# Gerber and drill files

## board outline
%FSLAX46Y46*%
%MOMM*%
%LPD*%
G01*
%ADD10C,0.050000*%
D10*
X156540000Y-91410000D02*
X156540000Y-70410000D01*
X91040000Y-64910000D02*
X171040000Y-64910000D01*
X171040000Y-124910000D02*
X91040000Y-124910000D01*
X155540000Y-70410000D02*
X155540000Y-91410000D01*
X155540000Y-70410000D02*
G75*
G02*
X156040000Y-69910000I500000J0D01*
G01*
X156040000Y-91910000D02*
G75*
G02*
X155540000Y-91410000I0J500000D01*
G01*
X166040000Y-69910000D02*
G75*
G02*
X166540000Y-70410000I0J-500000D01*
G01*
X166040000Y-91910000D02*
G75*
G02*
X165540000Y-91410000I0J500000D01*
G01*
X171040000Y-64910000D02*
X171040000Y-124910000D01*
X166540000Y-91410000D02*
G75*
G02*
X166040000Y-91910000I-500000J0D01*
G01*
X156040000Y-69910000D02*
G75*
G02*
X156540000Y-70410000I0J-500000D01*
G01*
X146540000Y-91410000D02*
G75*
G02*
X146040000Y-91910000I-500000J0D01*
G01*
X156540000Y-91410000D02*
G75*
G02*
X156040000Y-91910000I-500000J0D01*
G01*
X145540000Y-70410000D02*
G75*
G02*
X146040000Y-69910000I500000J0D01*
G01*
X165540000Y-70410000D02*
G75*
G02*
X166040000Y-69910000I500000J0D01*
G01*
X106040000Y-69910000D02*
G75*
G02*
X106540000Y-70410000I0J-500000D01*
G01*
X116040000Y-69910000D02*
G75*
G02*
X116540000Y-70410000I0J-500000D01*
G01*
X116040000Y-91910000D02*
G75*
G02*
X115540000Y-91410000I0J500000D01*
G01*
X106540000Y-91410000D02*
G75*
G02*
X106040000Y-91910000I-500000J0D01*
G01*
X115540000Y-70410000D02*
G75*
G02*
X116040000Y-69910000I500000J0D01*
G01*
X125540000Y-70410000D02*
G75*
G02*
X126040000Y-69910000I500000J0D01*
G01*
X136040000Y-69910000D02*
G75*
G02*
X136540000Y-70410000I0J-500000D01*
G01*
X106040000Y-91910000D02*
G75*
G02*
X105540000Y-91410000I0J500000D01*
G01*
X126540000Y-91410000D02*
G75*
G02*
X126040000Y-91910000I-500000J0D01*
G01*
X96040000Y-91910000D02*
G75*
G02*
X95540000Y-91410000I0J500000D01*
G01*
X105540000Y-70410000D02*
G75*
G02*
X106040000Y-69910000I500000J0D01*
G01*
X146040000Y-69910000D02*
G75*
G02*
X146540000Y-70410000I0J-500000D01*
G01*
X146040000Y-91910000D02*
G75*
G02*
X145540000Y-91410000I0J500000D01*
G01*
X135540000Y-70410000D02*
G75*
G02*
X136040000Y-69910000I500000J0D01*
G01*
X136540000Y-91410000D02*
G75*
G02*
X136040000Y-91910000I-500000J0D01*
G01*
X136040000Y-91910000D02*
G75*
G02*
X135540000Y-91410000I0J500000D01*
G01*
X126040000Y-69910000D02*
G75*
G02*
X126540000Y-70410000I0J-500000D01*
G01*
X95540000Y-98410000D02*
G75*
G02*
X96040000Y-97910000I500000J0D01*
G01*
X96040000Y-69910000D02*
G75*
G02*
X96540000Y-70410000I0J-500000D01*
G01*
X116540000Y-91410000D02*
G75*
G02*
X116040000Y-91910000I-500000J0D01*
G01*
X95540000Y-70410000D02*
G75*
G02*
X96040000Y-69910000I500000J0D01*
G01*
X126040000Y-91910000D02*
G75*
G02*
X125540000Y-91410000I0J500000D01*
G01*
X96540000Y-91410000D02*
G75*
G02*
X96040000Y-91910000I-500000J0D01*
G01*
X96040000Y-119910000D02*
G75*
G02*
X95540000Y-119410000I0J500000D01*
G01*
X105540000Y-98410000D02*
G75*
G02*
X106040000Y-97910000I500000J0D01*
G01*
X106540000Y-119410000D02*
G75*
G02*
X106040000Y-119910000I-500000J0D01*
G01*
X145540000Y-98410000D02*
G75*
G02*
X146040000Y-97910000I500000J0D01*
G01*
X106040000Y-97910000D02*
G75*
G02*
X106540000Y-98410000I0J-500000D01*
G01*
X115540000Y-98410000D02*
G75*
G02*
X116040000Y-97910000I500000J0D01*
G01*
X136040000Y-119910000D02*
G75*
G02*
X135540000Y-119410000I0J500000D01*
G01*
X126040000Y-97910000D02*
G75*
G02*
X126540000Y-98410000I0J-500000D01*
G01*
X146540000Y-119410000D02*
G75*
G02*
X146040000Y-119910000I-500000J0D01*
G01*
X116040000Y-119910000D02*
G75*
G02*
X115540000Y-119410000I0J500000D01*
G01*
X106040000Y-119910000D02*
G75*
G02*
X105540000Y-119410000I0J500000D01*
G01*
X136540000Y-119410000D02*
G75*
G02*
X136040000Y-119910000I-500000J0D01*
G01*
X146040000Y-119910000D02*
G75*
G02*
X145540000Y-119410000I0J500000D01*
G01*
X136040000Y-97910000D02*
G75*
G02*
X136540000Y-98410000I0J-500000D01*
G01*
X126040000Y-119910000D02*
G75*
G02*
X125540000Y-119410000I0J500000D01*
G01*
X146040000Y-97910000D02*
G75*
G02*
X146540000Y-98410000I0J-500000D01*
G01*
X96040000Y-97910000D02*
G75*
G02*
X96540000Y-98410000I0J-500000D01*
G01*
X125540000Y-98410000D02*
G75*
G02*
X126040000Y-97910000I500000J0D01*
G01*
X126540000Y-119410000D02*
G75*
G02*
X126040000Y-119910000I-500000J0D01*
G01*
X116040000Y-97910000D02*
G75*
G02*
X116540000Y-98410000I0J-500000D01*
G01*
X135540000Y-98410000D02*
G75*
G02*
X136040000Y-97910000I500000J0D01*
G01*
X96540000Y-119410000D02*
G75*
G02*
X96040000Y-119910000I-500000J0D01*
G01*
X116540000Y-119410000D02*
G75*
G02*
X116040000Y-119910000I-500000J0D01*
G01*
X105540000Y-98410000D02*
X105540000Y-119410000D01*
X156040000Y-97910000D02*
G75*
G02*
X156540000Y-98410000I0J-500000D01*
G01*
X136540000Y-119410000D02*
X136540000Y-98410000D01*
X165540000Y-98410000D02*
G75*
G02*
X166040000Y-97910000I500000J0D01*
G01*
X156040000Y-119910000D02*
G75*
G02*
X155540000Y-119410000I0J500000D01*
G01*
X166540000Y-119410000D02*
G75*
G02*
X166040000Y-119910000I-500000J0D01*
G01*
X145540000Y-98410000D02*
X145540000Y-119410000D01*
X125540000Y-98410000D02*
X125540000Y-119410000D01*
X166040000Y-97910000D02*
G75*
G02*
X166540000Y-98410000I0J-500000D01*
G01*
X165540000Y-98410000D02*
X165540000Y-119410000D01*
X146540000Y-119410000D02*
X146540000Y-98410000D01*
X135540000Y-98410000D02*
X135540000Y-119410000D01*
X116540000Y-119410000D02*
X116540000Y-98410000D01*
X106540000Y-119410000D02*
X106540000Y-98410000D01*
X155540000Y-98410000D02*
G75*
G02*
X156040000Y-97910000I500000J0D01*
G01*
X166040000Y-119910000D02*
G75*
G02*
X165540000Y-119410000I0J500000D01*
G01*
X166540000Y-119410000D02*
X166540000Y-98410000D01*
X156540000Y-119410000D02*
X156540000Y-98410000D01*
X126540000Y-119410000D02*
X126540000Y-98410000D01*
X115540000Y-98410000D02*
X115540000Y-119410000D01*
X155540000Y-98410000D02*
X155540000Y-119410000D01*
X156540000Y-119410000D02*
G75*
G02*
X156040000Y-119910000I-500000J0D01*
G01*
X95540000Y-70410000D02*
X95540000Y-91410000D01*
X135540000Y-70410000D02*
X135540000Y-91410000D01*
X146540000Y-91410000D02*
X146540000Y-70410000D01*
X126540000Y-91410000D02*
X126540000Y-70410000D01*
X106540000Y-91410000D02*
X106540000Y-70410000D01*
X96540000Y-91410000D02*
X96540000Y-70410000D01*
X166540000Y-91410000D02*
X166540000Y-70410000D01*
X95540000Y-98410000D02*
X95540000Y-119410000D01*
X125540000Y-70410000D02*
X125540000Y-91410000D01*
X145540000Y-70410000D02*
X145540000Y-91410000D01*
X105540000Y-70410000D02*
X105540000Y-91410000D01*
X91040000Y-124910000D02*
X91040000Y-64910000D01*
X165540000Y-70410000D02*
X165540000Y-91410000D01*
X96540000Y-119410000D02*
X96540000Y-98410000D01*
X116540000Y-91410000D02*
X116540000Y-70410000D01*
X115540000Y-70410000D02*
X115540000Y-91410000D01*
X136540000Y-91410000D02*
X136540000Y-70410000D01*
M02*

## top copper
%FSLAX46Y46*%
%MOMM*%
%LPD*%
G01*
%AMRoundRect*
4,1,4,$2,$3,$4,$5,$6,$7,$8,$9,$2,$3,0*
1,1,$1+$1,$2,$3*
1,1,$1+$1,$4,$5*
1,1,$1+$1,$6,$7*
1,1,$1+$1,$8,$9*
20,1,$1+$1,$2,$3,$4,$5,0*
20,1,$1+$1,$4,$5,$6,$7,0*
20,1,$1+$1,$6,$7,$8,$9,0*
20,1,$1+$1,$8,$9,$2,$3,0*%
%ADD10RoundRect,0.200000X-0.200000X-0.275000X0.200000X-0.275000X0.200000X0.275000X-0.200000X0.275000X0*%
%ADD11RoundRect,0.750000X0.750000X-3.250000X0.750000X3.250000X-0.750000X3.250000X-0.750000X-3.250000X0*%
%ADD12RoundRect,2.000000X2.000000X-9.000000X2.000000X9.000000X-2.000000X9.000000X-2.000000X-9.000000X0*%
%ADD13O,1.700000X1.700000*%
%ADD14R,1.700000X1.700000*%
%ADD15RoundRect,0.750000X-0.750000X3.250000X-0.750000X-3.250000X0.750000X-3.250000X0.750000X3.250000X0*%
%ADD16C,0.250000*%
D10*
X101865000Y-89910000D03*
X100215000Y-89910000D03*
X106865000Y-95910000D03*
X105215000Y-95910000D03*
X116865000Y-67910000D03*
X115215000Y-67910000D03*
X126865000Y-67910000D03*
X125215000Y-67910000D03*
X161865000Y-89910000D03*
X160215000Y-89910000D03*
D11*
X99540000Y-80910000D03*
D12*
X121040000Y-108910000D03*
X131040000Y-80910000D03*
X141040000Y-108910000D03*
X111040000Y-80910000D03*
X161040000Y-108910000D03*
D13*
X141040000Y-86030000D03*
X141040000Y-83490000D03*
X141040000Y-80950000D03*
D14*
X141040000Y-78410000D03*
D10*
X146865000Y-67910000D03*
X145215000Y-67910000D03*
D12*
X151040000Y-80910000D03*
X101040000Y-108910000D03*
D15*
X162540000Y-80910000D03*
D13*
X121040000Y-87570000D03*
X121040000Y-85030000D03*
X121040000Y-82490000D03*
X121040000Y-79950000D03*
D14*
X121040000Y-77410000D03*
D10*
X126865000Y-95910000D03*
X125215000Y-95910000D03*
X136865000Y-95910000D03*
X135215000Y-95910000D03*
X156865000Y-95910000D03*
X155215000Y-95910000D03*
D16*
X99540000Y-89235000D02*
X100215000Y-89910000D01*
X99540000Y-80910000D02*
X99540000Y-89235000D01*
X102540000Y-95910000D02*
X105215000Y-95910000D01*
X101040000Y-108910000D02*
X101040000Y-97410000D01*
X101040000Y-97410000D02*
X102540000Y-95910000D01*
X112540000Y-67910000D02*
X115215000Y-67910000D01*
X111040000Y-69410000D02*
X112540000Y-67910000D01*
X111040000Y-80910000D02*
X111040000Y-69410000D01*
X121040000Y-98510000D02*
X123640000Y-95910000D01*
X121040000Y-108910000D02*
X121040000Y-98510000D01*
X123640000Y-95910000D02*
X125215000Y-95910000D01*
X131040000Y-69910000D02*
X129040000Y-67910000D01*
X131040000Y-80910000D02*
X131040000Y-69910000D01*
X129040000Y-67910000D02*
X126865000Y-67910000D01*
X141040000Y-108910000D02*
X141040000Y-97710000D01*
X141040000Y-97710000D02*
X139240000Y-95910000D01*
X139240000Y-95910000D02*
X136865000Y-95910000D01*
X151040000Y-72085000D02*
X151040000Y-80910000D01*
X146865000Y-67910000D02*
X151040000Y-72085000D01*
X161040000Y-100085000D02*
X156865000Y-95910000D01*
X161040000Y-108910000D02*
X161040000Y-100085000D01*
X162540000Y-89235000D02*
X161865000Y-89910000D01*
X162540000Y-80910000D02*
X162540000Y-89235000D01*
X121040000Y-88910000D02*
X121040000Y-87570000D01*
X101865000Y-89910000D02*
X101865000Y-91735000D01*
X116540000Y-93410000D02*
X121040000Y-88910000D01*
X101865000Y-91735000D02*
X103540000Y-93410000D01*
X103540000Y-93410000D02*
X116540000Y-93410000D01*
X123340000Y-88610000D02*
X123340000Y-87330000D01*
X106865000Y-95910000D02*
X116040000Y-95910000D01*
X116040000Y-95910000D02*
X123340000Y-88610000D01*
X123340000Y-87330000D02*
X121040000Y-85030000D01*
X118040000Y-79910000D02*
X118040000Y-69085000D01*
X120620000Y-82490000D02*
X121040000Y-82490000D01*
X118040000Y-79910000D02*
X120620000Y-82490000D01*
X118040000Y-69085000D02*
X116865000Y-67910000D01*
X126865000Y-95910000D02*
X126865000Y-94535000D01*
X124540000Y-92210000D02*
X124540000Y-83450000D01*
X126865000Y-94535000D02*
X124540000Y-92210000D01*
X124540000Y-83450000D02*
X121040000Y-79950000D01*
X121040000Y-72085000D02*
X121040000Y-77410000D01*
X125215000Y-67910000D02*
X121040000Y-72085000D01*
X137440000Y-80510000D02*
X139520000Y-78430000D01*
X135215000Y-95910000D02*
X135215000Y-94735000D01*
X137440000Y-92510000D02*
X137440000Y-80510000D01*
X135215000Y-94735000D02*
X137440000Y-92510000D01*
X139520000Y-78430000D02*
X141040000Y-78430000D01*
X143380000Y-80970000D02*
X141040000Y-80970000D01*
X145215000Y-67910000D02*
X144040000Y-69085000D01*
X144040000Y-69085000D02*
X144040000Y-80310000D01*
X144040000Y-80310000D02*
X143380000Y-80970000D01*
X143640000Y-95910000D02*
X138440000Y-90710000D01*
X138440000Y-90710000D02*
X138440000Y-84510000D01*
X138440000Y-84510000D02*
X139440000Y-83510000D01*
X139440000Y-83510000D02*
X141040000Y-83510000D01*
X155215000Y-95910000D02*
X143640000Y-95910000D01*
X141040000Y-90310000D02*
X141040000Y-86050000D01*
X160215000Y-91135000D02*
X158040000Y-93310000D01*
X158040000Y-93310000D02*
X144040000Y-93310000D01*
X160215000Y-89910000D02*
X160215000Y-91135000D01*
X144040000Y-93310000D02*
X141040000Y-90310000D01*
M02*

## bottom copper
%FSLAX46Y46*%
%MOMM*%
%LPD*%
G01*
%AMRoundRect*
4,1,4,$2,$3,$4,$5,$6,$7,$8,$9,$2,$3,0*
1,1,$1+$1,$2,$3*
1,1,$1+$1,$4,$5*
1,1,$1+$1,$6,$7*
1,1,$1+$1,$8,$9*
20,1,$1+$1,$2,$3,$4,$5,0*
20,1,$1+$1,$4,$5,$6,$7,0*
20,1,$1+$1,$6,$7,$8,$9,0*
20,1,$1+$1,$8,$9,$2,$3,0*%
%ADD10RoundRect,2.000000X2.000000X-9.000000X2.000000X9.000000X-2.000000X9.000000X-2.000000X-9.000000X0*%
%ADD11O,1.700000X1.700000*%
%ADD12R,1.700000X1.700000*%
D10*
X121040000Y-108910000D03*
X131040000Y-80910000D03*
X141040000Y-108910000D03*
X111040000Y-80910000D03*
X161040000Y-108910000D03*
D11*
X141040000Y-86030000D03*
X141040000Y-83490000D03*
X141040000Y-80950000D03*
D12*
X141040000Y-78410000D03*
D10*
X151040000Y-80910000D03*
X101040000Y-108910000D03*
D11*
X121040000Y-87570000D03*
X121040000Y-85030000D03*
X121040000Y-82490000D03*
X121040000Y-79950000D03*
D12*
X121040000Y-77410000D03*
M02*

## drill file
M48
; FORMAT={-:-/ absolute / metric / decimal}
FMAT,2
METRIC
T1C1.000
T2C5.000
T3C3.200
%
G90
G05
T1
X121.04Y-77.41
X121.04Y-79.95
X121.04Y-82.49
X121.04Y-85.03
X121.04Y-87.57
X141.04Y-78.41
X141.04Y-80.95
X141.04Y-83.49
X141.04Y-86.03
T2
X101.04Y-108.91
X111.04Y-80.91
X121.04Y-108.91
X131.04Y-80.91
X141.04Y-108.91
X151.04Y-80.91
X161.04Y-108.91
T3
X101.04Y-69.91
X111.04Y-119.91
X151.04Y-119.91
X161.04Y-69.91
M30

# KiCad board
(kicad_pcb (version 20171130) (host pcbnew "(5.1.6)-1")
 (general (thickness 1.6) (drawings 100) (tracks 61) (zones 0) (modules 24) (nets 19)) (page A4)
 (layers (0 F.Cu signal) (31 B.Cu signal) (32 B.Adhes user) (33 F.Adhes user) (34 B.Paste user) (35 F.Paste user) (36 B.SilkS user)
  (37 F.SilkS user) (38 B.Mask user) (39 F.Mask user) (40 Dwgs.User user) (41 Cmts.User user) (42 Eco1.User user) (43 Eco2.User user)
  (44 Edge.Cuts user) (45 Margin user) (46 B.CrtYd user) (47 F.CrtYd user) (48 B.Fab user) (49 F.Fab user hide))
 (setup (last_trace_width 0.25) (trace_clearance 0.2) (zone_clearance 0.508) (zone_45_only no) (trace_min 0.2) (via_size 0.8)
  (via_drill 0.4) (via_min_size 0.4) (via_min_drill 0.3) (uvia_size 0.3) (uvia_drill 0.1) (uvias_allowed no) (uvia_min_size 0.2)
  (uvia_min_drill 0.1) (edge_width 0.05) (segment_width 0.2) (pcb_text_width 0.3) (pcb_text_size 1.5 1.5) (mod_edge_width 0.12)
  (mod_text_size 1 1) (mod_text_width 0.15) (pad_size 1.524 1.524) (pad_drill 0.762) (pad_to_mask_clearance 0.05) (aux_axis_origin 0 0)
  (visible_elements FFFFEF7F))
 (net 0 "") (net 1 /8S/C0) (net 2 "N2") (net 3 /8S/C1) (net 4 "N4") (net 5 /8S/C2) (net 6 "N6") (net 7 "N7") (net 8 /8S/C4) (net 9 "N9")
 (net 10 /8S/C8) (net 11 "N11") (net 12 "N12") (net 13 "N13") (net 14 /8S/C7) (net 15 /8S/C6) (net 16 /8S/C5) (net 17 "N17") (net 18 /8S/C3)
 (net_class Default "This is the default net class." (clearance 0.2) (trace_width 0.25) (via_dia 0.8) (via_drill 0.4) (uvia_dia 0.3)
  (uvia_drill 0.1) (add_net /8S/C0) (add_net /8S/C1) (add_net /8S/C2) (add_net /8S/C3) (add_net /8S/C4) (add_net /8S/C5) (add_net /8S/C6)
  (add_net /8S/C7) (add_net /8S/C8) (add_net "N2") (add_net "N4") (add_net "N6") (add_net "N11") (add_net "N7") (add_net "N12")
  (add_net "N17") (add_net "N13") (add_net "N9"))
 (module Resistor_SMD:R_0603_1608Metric (layer F.Cu) (at 101.04 89.91)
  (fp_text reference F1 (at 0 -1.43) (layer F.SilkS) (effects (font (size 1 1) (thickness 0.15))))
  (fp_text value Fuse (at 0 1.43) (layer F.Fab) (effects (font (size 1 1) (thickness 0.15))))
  (pad 2 smd roundrect (at 0.825 0) (size 0.8 0.95) (layers F.Cu F.Paste F.Mask) (roundrect_rratio 0.25) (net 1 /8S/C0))
  (pad 1 smd roundrect (at -0.825 0) (size 0.8 0.95) (layers F.Cu F.Paste F.Mask) (roundrect_rratio 0.25) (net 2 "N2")))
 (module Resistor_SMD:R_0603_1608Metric (layer F.Cu) (at 106.04 95.91)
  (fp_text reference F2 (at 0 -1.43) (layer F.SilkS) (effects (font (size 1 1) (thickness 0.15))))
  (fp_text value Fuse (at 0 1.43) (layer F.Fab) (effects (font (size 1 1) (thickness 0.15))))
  (pad 2 smd roundrect (at 0.825 0) (size 0.8 0.95) (layers F.Cu F.Paste F.Mask) (roundrect_rratio 0.25) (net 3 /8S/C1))
  (pad 1 smd roundrect (at -0.825 0) (size 0.8 0.95) (layers F.Cu F.Paste F.Mask) (roundrect_rratio 0.25) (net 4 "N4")))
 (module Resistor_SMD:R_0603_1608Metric (layer F.Cu) (at 116.04 67.91)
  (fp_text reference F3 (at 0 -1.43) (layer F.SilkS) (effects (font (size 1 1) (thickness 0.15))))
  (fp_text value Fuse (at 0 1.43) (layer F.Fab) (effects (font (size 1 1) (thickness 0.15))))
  (pad 2 smd roundrect (at 0.825 0) (size 0.8 0.95) (layers F.Cu F.Paste F.Mask) (roundrect_rratio 0.25) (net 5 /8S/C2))
  (pad 1 smd roundrect (at -0.825 0) (size 0.8 0.95) (layers F.Cu F.Paste F.Mask) (roundrect_rratio 0.25) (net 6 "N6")))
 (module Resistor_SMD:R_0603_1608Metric (layer F.Cu) (at 126.04 67.91)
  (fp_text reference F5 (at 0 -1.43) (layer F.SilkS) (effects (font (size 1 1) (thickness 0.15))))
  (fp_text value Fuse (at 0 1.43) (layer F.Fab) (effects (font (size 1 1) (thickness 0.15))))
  (pad 2 smd roundrect (at 0.825 0) (size 0.8 0.95) (layers F.Cu F.Paste F.Mask) (roundrect_rratio 0.25) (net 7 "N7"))
  (pad 1 smd roundrect (at -0.825 0) (size 0.8 0.95) (layers F.Cu F.Paste F.Mask) (roundrect_rratio 0.25) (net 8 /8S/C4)))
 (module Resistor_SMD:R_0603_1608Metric (layer F.Cu) (at 161.04 89.91)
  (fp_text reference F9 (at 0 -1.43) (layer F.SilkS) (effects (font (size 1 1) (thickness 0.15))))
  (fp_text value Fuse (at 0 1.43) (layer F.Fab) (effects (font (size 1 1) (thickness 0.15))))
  (pad 2 smd roundrect (at 0.825 0) (size 0.8 0.95) (layers F.Cu F.Paste F.Mask) (roundrect_rratio 0.25) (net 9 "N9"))
  (pad 1 smd roundrect (at -0.825 0) (size 0.8 0.95) (layers F.Cu F.Paste F.Mask) (roundrect_rratio 0.25) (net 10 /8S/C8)))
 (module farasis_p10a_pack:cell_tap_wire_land (layer F.Cu) (at 99.54 80.91 90)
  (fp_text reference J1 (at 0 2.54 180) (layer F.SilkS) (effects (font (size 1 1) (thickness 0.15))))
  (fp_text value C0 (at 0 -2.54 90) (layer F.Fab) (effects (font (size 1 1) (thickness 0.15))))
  (pad 1 smd roundrect (at 0 0 90) (size 8 3) (layers F.Cu F.Paste F.Mask) (roundrect_rratio 0.25) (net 2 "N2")))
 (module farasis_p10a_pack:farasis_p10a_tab (layer F.Cu) (at 121.04 108.91 90)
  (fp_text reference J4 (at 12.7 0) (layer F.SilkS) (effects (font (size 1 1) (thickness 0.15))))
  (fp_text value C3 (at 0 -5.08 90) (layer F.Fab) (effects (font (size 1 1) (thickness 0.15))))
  (pad 1 thru_hole roundrect (at 0 0 90) (size 22 8) (drill 5) (layers *.Cu *.Mask) (roundrect_rratio 0.25) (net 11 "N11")))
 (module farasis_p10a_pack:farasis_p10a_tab (layer F.Cu) (at 131.04 80.91 90)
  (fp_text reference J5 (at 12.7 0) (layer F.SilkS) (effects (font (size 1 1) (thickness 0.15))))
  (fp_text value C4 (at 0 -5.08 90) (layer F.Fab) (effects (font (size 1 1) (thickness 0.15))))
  (pad 1 thru_hole roundrect (at 0 0 90) (size 22 8) (drill 5) (layers *.Cu *.Mask) (roundrect_rratio 0.25) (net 7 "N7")))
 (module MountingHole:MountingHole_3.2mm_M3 (layer F.Cu) (at 101.04 69.91 180)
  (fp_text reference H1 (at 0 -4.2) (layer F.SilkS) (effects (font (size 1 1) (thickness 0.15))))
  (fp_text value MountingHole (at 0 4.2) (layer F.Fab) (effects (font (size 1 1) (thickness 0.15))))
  (pad 1 np_thru_hole circle (at 0 0 180) (size 3.2 3.2) (drill 3.2) (layers *.Cu *.Mask)))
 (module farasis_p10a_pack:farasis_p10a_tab (layer F.Cu) (at 141.04 108.91 90)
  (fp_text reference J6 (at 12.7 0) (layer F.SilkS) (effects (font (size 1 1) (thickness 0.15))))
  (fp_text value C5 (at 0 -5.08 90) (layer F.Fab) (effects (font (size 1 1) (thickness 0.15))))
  (pad 1 thru_hole roundrect (at 0 0 90) (size 22 8) (drill 5) (layers *.Cu *.Mask) (roundrect_rratio 0.25) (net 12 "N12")))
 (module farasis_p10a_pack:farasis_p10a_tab (layer F.Cu) (at 111.04 80.91 90)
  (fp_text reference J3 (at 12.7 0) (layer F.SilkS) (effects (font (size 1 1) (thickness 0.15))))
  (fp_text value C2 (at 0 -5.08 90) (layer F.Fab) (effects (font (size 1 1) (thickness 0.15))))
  (pad 1 thru_hole roundrect (at 0 0 90) (size 22 8) (drill 5) (layers *.Cu *.Mask) (roundrect_rratio 0.25) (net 6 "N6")))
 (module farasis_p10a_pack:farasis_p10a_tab (layer F.Cu) (at 161.04 108.91 90)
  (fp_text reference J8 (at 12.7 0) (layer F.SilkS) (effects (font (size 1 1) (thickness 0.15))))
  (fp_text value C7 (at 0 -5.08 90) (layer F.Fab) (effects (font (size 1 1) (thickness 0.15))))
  (pad 1 thru_hole roundrect (at 0 0 90) (size 22 8) (drill 5) (layers *.Cu *.Mask) (roundrect_rratio 0.25) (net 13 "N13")))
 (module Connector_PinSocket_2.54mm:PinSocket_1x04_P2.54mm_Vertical (layer F.Cu) (at 141.04 78.41)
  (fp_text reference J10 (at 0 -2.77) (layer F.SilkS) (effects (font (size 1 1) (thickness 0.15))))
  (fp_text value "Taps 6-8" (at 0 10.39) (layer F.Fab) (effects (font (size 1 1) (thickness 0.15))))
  (pad 4 thru_hole oval (at 0 7.62) (size 1.7 1.7) (drill 1) (layers *.Cu *.Mask) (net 10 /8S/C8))
  (pad 3 thru_hole oval (at 0 5.08) (size 1.7 1.7) (drill 1) (layers *.Cu *.Mask) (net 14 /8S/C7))
  (pad 2 thru_hole oval (at 0 2.54) (size 1.7 1.7) (drill 1) (layers *.Cu *.Mask) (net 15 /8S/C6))
  (pad 1 thru_hole rect (at 0 0) (size 1.7 1.7) (drill 1) (layers *.Cu *.Mask) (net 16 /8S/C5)))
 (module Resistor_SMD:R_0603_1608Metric (layer F.Cu) (at 146.04 67.91)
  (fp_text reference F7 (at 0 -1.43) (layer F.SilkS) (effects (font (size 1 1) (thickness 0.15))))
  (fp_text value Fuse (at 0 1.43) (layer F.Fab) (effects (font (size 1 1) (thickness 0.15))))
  (pad 2 smd roundrect (at 0.825 0) (size 0.8 0.95) (layers F.Cu F.Paste F.Mask) (roundrect_rratio 0.25) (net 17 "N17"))
  (pad 1 smd roundrect (at -0.825 0) (size 0.8 0.95) (layers F.Cu F.Paste F.Mask) (roundrect_rratio 0.25) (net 15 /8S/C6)))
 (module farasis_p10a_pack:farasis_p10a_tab (layer F.Cu) (at 151.04 80.91 90)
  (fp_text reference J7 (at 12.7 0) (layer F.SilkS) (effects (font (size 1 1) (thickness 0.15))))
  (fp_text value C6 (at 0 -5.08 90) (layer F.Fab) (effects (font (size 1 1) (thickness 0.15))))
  (pad 1 thru_hole roundrect (at 0 0 90) (size 22 8) (drill 5) (layers *.Cu *.Mask) (roundrect_rratio 0.25) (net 17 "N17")))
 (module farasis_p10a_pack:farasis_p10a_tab (layer F.Cu) (at 101.04 108.91 90)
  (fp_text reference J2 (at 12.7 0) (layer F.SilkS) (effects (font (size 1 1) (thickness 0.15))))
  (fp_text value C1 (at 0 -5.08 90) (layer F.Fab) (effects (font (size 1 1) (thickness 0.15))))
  (pad 1 thru_hole roundrect (at 0 0 90) (size 22 8) (drill 5) (layers *.Cu *.Mask) (roundrect_rratio 0.25) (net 4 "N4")))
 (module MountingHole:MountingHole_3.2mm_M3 (layer F.Cu) (at 151.04 119.91)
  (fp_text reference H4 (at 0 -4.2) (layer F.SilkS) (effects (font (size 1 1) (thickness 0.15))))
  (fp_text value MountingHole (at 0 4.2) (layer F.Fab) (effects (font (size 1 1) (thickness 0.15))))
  (pad 1 np_thru_hole circle (at 0 0) (size 3.2 3.2) (drill 3.2) (layers *.Cu *.Mask)))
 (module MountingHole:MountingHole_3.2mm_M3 (layer F.Cu) (at 161.04 69.91 180)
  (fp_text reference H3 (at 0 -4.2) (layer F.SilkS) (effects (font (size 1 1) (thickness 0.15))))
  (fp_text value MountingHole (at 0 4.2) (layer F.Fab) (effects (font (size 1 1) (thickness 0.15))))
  (pad 1 np_thru_hole circle (at 0 0 180) (size 3.2 3.2) (drill 3.2) (layers *.Cu *.Mask)))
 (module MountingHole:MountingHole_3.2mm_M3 (layer F.Cu) (at 111.04 119.91)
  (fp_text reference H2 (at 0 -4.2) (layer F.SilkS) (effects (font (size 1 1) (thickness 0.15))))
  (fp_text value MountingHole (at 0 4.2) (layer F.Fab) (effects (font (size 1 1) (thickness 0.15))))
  (pad 1 np_thru_hole circle (at 0 0) (size 3.2 3.2) (drill 3.2) (layers *.Cu *.Mask)))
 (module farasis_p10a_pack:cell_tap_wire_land (layer F.Cu) (at 162.54 80.91 270)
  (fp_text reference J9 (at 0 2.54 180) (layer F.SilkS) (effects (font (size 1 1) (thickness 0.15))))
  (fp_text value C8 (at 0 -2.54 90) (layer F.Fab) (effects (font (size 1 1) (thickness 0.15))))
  (pad 1 smd roundrect (at 0 0 270) (size 8 3) (layers F.Cu F.Paste F.Mask) (roundrect_rratio 0.25) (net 9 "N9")))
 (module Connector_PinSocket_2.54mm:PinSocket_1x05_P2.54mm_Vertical (layer F.Cu) (at 121.04 77.41)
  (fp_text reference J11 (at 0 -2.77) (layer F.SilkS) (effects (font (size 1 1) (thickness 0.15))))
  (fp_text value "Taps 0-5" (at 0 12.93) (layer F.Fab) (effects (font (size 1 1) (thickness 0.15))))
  (pad 5 thru_hole oval (at 0 10.16) (size 1.7 1.7) (drill 1) (layers *.Cu *.Mask) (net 1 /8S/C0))
  (pad 4 thru_hole oval (at 0 7.62) (size 1.7 1.7) (drill 1) (layers *.Cu *.Mask) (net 3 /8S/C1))
  (pad 3 thru_hole oval (at 0 5.08) (size 1.7 1.7) (drill 1) (layers *.Cu *.Mask) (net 5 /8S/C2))
  (pad 2 thru_hole oval (at 0 2.54) (size 1.7 1.7) (drill 1) (layers *.Cu *.Mask) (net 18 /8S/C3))
  (pad 1 thru_hole rect (at 0 0) (size 1.7 1.7) (drill 1) (layers *.Cu *.Mask) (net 8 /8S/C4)))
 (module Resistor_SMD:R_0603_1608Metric (layer F.Cu) (at 126.04 95.91)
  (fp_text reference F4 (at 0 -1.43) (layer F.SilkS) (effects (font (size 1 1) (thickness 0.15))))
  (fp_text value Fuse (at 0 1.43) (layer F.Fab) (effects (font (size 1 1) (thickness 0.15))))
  (pad 2 smd roundrect (at 0.825 0) (size 0.8 0.95) (layers F.Cu F.Paste F.Mask) (roundrect_rratio 0.25) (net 18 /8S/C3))
  (pad 1 smd roundrect (at -0.825 0) (size 0.8 0.95) (layers F.Cu F.Paste F.Mask) (roundrect_rratio 0.25) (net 11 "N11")))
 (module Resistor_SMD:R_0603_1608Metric (layer F.Cu) (at 136.04 95.91)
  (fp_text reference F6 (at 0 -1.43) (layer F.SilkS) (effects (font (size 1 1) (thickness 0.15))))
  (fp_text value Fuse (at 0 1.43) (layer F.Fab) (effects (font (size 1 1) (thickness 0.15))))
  (pad 2 smd roundrect (at 0.825 0) (size 0.8 0.95) (layers F.Cu F.Paste F.Mask) (roundrect_rratio 0.25) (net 12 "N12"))
  (pad 1 smd roundrect (at -0.825 0) (size 0.8 0.95) (layers F.Cu F.Paste F.Mask) (roundrect_rratio 0.25) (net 16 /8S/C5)))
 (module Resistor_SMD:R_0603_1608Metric (layer F.Cu) (at 156.04 95.91)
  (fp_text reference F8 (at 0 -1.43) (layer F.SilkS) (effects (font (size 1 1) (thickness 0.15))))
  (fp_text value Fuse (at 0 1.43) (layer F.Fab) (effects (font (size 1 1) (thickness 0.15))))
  (pad 2 smd roundrect (at 0.825 0) (size 0.8 0.95) (layers F.Cu F.Paste F.Mask) (roundrect_rratio 0.25) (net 13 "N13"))
  (pad 1 smd roundrect (at -0.825 0) (size 0.8 0.95) (layers F.Cu F.Paste F.Mask) (roundrect_rratio 0.25) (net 14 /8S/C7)))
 (gr_line (start 156.54 91.41) (end 156.54 70.41) (layer Edge.Cuts) (width 0.05))
 (gr_line (start 91.04 64.91) (end 171.04 64.91) (layer Edge.Cuts) (width 0.05))
 (gr_line (start 171.04 124.91) (end 91.04 124.91) (layer Edge.Cuts) (width 0.05))
 (gr_line (start 155.54 70.41) (end 155.54 91.41) (layer Edge.Cuts) (width 0.05))
 (gr_arc (start 156.04 70.41) (end 156.04 69.91) (angle -90) (layer Edge.Cuts) (width 0.05))
 (gr_arc (start 156.04 91.41) (end 155.54 91.41) (angle -90) (layer Edge.Cuts) (width 0.05))
 (gr_arc (start 166.04 70.41) (end 166.54 70.41) (angle -90) (layer Edge.Cuts) (width 0.05))
 (gr_arc (start 166.04 91.41) (end 165.54 91.41) (angle -90) (layer Edge.Cuts) (width 0.05))
 (gr_line (start 171.04 64.91) (end 171.04 124.91) (layer Edge.Cuts) (width 0.05))
 (gr_arc (start 166.04 91.41) (end 166.04 91.91) (angle -90) (layer Edge.Cuts) (width 0.05))
 (gr_arc (start 156.04 70.41) (end 156.54 70.41) (angle -90) (layer Edge.Cuts) (width 0.05))
 (gr_arc (start 146.04 91.41) (end 146.04 91.91) (angle -90) (layer Edge.Cuts) (width 0.05))
 (gr_arc (start 156.04 91.41) (end 156.04 91.91) (angle -90) (layer Edge.Cuts) (width 0.05))
 (gr_arc (start 146.04 70.41) (end 146.04 69.91) (angle -90) (layer Edge.Cuts) (width 0.05))
 (gr_arc (start 166.04 70.41) (end 166.04 69.91) (angle -90) (layer Edge.Cuts) (width 0.05))
 (gr_arc (start 106.04 70.41) (end 106.54 70.41) (angle -90) (layer Edge.Cuts) (width 0.05))
 (gr_arc (start 116.04 70.41) (end 116.54 70.41) (angle -90) (layer Edge.Cuts) (width 0.05))
 (gr_arc (start 116.04 91.41) (end 115.54 91.41) (angle -90) (layer Edge.Cuts) (width 0.05))
 (gr_arc (start 106.04 91.41) (end 106.04 91.91) (angle -90) (layer Edge.Cuts) (width 0.05))
 (gr_arc (start 116.04 70.41) (end 116.04 69.91) (angle -90) (layer Edge.Cuts) (width 0.05))
 (gr_arc (start 126.04 70.41) (end 126.04 69.91) (angle -90) (layer Edge.Cuts) (width 0.05))
 (gr_arc (start 136.04 70.41) (end 136.54 70.41) (angle -90) (layer Edge.Cuts) (width 0.05))
 (gr_arc (start 106.04 91.41) (end 105.54 91.41) (angle -90) (layer Edge.Cuts) (width 0.05))
 (gr_arc (start 126.04 91.41) (end 126.04 91.91) (angle -90) (layer Edge.Cuts) (width 0.05))
 (gr_arc (start 96.04 91.41) (end 95.54 91.41) (angle -90) (layer Edge.Cuts) (width 0.05))
 (gr_arc (start 106.04 70.41) (end 106.04 69.91) (angle -90) (layer Edge.Cuts) (width 0.05))
 (gr_arc (start 146.04 70.41) (end 146.54 70.41) (angle -90) (layer Edge.Cuts) (width 0.05))
 (gr_arc (start 146.04 91.41) (end 145.54 91.41) (angle -90) (layer Edge.Cuts) (width 0.05))
 (gr_arc (start 136.04 70.41) (end 136.04 69.91) (angle -90) (layer Edge.Cuts) (width 0.05))
 (gr_arc (start 136.04 91.41) (end 136.04 91.91) (angle -90) (layer Edge.Cuts) (width 0.05))
 (gr_arc (start 136.04 91.41) (end 135.54 91.41) (angle -90) (layer Edge.Cuts) (width 0.05))
 (gr_arc (start 126.04 70.41) (end 126.54 70.41) (angle -90) (layer Edge.Cuts) (width 0.05))
 (gr_arc (start 96.04 98.41) (end 96.04 97.91) (angle -90) (layer Edge.Cuts) (width 0.05))
 (gr_arc (start 96.04 70.41) (end 96.54 70.41) (angle -90) (layer Edge.Cuts) (width 0.05))
 (gr_arc (start 116.04 91.41) (end 116.04 91.91) (angle -90) (layer Edge.Cuts) (width 0.05))
 (gr_arc (start 96.04 70.41) (end 96.04 69.91) (angle -90) (layer Edge.Cuts) (width 0.05))
 (gr_arc (start 126.04 91.41) (end 125.54 91.41) (angle -90) (layer Edge.Cuts) (width 0.05))
 (gr_arc (start 96.04 91.41) (end 96.04 91.91) (angle -90) (layer Edge.Cuts) (width 0.05))
 (gr_arc (start 96.04 119.41) (end 95.54 119.41) (angle -90) (layer Edge.Cuts) (width 0.05))
 (gr_arc (start 106.04 98.41) (end 106.04 97.91) (angle -90) (layer Edge.Cuts) (width 0.05))
 (gr_arc (start 106.04 119.41) (end 106.04 119.91) (angle -90) (layer Edge.Cuts) (width 0.05))
 (gr_arc (start 146.04 98.41) (end 146.04 97.91) (angle -90) (layer Edge.Cuts) (width 0.05))
 (gr_arc (start 106.04 98.41) (end 106.54 98.41) (angle -90) (layer Edge.Cuts) (width 0.05))
 (gr_arc (start 116.04 98.41) (end 116.04 97.91) (angle -90) (layer Edge.Cuts) (width 0.05))
 (gr_arc (start 136.04 119.41) (end 135.54 119.41) (angle -90) (layer Edge.Cuts) (width 0.05))
 (gr_arc (start 126.04 98.41) (end 126.54 98.41) (angle -90) (layer Edge.Cuts) (width 0.05))
 (gr_arc (start 146.04 119.41) (end 146.04 119.91) (angle -90) (layer Edge.Cuts) (width 0.05))
 (gr_arc (start 116.04 119.41) (end 115.54 119.41) (angle -90) (layer Edge.Cuts) (width 0.05))
 (gr_arc (start 106.04 119.41) (end 105.54 119.41) (angle -90) (layer Edge.Cuts) (width 0.05))
 (gr_arc (start 136.04 119.41) (end 136.04 119.91) (angle -90) (layer Edge.Cuts) (width 0.05))
 (gr_arc (start 146.04 119.41) (end 145.54 119.41) (angle -90) (layer Edge.Cuts) (width 0.05))
 (gr_arc (start 136.04 98.41) (end 136.54 98.41) (angle -90) (layer Edge.Cuts) (width 0.05))
 (gr_arc (start 126.04 119.41) (end 125.54 119.41) (angle -90) (layer Edge.Cuts) (width 0.05))
 (gr_arc (start 146.04 98.41) (end 146.54 98.41) (angle -90) (layer Edge.Cuts) (width 0.05))
 (gr_arc (start 96.04 98.41) (end 96.54 98.41) (angle -90) (layer Edge.Cuts) (width 0.05))
 (gr_arc (start 126.04 98.41) (end 126.04 97.91) (angle -90) (layer Edge.Cuts) (width 0.05))
 (gr_arc (start 126.04 119.41) (end 126.04 119.91) (angle -90) (layer Edge.Cuts) (width 0.05))
 (gr_arc (start 116.04 98.41) (end 116.54 98.41) (angle -90) (layer Edge.Cuts) (width 0.05))
 (gr_arc (start 136.04 98.41) (end 136.04 97.91) (angle -90) (layer Edge.Cuts) (width 0.05))
 (gr_arc (start 96.04 119.41) (end 96.04 119.91) (angle -90) (layer Edge.Cuts) (width 0.05))
 (gr_arc (start 116.04 119.41) (end 116.04 119.91) (angle -90) (layer Edge.Cuts) (width 0.05))
 (gr_line (start 105.54 98.41) (end 105.54 119.41) (layer Edge.Cuts) (width 0.05))
 (gr_arc (start 156.04 98.41) (end 156.54 98.41) (angle -90) (layer Edge.Cuts) (width 0.05))
 (gr_line (start 136.54 119.41) (end 136.54 98.41) (layer Edge.Cuts) (width 0.05))
 (gr_arc (start 166.04 98.41) (end 166.04 97.91) (angle -90) (layer Edge.Cuts) (width 0.05))
 (gr_arc (start 156.04 119.41) (end 155.54 119.41) (angle -90) (layer Edge.Cuts) (width 0.05))
 (gr_arc (start 166.04 119.41) (end 166.04 119.91) (angle -90) (layer Edge.Cuts) (width 0.05))
 (gr_line (start 145.54 98.41) (end 145.54 119.41) (layer Edge.Cuts) (width 0.05))
 (gr_line (start 125.54 98.41) (end 125.54 119.41) (layer Edge.Cuts) (width 0.05))
 (gr_arc (start 166.04 98.41) (end 166.54 98.41) (angle -90) (layer Edge.Cuts) (width 0.05))
 (gr_line (start 165.54 98.41) (end 165.54 119.41) (layer Edge.Cuts) (width 0.05))
 (gr_line (start 146.54 119.41) (end 146.54 98.41) (layer Edge.Cuts) (width 0.05))
 (gr_line (start 135.54 98.41) (end 135.54 119.41) (layer Edge.Cuts) (width 0.05))
 (gr_line (start 116.54 119.41) (end 116.54 98.41) (layer Edge.Cuts) (width 0.05))
 (gr_line (start 106.54 119.41) (end 106.54 98.41) (layer Edge.Cuts) (width 0.05))
 (gr_arc (start 156.04 98.41) (end 156.04 97.91) (angle -90) (layer Edge.Cuts) (width 0.05))
 (gr_arc (start 166.04 119.41) (end 165.54 119.41) (angle -90) (layer Edge.Cuts) (width 0.05))
 (gr_line (start 166.54 119.41) (end 166.54 98.41) (layer Edge.Cuts) (width 0.05))
 (gr_line (start 156.54 119.41) (end 156.54 98.41) (layer Edge.Cuts) (width 0.05))
 (gr_line (start 126.54 119.41) (end 126.54 98.41) (layer Edge.Cuts) (width 0.05))
 (gr_line (start 115.54 98.41) (end 115.54 119.41) (layer Edge.Cuts) (width 0.05))
 (gr_line (start 155.54 98.41) (end 155.54 119.41) (layer Edge.Cuts) (width 0.05))
 (gr_arc (start 156.04 119.41) (end 156.04 119.91) (angle -90) (layer Edge.Cuts) (width 0.05))
 (gr_line (start 95.54 70.41) (end 95.54 91.41) (layer Edge.Cuts) (width 0.05))
 (gr_line (start 135.54 70.41) (end 135.54 91.41) (layer Edge.Cuts) (width 0.05))
 (gr_line (start 146.54 91.41) (end 146.54 70.41) (layer Edge.Cuts) (width 0.05))
 (gr_line (start 126.54 91.41) (end 126.54 70.41) (layer Edge.Cuts) (width 0.05))
 (gr_line (start 106.54 91.41) (end 106.54 70.41) (layer Edge.Cuts) (width 0.05))
 (gr_line (start 96.54 91.41) (end 96.54 70.41) (layer Edge.Cuts) (width 0.05))
 (gr_line (start 166.54 91.41) (end 166.54 70.41) (layer Edge.Cuts) (width 0.05))
 (gr_line (start 95.54 98.41) (end 95.54 119.41) (layer Edge.Cuts) (width 0.05))
 (gr_line (start 125.54 70.41) (end 125.54 91.41) (layer Edge.Cuts) (width 0.05))
 (gr_line (start 145.54 70.41) (end 145.54 91.41) (layer Edge.Cuts) (width 0.05))
 (gr_line (start 105.54 70.41) (end 105.54 91.41) (layer Edge.Cuts) (width 0.05))
 (gr_line (start 91.04 124.91) (end 91.04 64.91) (layer Edge.Cuts) (width 0.05))
 (gr_line (start 165.54 70.41) (end 165.54 91.41) (layer Edge.Cuts) (width 0.05))
 (gr_line (start 96.54 119.41) (end 96.54 98.41) (layer Edge.Cuts) (width 0.05))
 (gr_line (start 116.54 91.41) (end 116.54 70.41) (layer Edge.Cuts) (width 0.05))
 (gr_line (start 115.54 70.41) (end 115.54 91.41) (layer Edge.Cuts) (width 0.05))
 (gr_line (start 136.54 91.41) (end 136.54 70.41) (layer Edge.Cuts) (width 0.05))
 (segment (start 99.54 89.235) (end 100.215 89.91) (width 0.25) (layer F.Cu) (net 2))
 (segment (start 99.54 80.91) (end 99.54 89.235) (width 0.25) (layer F.Cu) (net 2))
 (segment (start 102.54 95.91) (end 105.215 95.91) (width 0.25) (layer F.Cu) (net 4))
 (segment (start 101.04 108.91) (end 101.04 97.41) (width 0.25) (layer F.Cu) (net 4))
 (segment (start 101.04 97.41) (end 102.54 95.91) (width 0.25) (layer F.Cu) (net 4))
 (segment (start 112.54 67.91) (end 115.215 67.91) (width 0.25) (layer F.Cu) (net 6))
 (segment (start 111.04 69.41) (end 112.54 67.91) (width 0.25) (layer F.Cu) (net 6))
 (segment (start 111.04 80.91) (end 111.04 69.41) (width 0.25) (layer F.Cu) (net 6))
 (segment (start 121.04 98.51) (end 123.64 95.91) (width 0.25) (layer F.Cu) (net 11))
 (segment (start 121.04 108.91) (end 121.04 98.51) (width 0.25) (layer F.Cu) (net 11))
 (segment (start 123.64 95.91) (end 125.215 95.91) (width 0.25) (layer F.Cu) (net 11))
 (segment (start 131.04 69.91) (end 129.04 67.91) (width 0.25) (layer F.Cu) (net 7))
 (segment (start 131.04 80.91) (end 131.04 69.91) (width 0.25) (layer F.Cu) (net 7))
 (segment (start 129.04 67.91) (end 126.865 67.91) (width 0.25) (layer F.Cu) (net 7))
 (segment (start 141.04 108.91) (end 141.04 97.71) (width 0.25) (layer F.Cu) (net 12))
 (segment (start 141.04 97.71) (end 139.24 95.91) (width 0.25) (layer F.Cu) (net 12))
 (segment (start 139.24 95.91) (end 136.865 95.91) (width 0.25) (layer F.Cu) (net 12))
 (segment (start 151.04 72.085) (end 151.04 80.91) (width 0.25) (layer F.Cu) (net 17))
 (segment (start 146.865 67.91) (end 151.04 72.085) (width 0.25) (layer F.Cu) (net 17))
 (segment (start 161.04 100.085) (end 156.865 95.91) (width 0.25) (layer F.Cu) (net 13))
 (segment (start 161.04 108.91) (end 161.04 100.085) (width 0.25) (layer F.Cu) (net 13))
 (segment (start 162.54 89.235) (end 161.865 89.91) (width 0.25) (layer F.Cu) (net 9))
 (segment (start 162.54 80.91) (end 162.54 89.235) (width 0.25) (layer F.Cu) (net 9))
 (segment (start 121.04 88.91) (end 121.04 87.57) (width 0.25) (layer F.Cu) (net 1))
 (segment (start 101.865 89.91) (end 101.865 91.735) (width 0.25) (layer F.Cu) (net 1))
 (segment (start 116.54 93.41) (end 121.04 88.91) (width 0.25) (layer F.Cu) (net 1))
 (segment (start 101.865 91.735) (end 103.54 93.41) (width 0.25) (layer F.Cu) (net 1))
 (segment (start 103.54 93.41) (end 116.54 93.41) (width 0.25) (layer F.Cu) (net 1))
 (segment (start 123.34 88.61) (end 123.34 87.33) (width 0.25) (layer F.Cu) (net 3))
 (segment (start 106.865 95.91) (end 116.04 95.91) (width 0.25) (layer F.Cu) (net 3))
 (segment (start 116.04 95.91) (end 123.34 88.61) (width 0.25) (layer F.Cu) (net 3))
 (segment (start 123.34 87.33) (end 121.04 85.03) (width 0.25) (layer F.Cu) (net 3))
 (segment (start 118.04 79.91) (end 118.04 69.085) (width 0.25) (layer F.Cu) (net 5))
 (segment (start 120.62 82.49) (end 121.04 82.49) (width 0.25) (layer F.Cu) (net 5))
 (segment (start 118.04 79.91) (end 120.62 82.49) (width 0.25) (layer F.Cu) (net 5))
 (segment (start 118.04 69.085) (end 116.865 67.91) (width 0.25) (layer F.Cu) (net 5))
 (segment (start 126.865 95.91) (end 126.865 94.535) (width 0.25) (layer F.Cu) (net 18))
 (segment (start 124.54 92.21) (end 124.54 83.45) (width 0.25) (layer F.Cu) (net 18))
 (segment (start 126.865 94.535) (end 124.54 92.21) (width 0.25) (layer F.Cu) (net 18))
 (segment (start 124.54 83.45) (end 121.04 79.95) (width 0.25) (layer F.Cu) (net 18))
 (segment (start 121.04 72.085) (end 121.04 77.41) (width 0.25) (layer F.Cu) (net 8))
 (segment (start 125.215 67.91) (end 121.04 72.085) (width 0.25) (layer F.Cu) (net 8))
 (segment (start 137.44 80.51) (end 139.52 78.43) (width 0.25) (layer F.Cu) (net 16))
 (segment (start 135.215 95.91) (end 135.215 94.735) (width 0.25) (layer F.Cu) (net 16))
 (segment (start 137.44 92.51) (end 137.44 80.51) (width 0.25) (layer F.Cu) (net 16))
 (segment (start 135.215 94.735) (end 137.44 92.51) (width 0.25) (layer F.Cu) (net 16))
 (segment (start 139.52 78.43) (end 141.04 78.43) (width 0.25) (layer F.Cu) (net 16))
 (segment (start 143.38 80.97) (end 141.04 80.97) (width 0.25) (layer F.Cu) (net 15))
 (segment (start 145.215 67.91) (end 144.04 69.085) (width 0.25) (layer F.Cu) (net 15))
 (segment (start 144.04 69.085) (end 144.04 80.31) (width 0.25) (layer F.Cu) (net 15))
 (segment (start 144.04 80.31) (end 143.38 80.97) (width 0.25) (layer F.Cu) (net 15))
 (segment (start 143.64 95.91) (end 138.44 90.71) (width 0.25) (layer F.Cu) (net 14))
 (segment (start 138.44 90.71) (end 138.44 84.51) (width 0.25) (layer F.Cu) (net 14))
 (segment (start 138.44 84.51) (end 139.44 83.51) (width 0.25) (layer F.Cu) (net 14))
 (segment (start 139.44 83.51) (end 141.04 83.51) (width 0.25) (layer F.Cu) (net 14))
 (segment (start 155.215 95.91) (end 143.64 95.91) (width 0.25) (layer F.Cu) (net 14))
 (segment (start 141.04 90.31) (end 141.04 86.05) (width 0.25) (layer F.Cu) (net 10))
 (segment (start 160.215 91.135) (end 158.04 93.31) (width 0.25) (layer F.Cu) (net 10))
 (segment (start 158.04 93.31) (end 144.04 93.31) (width 0.25) (layer F.Cu) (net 10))
 (segment (start 160.215 89.91) (end 160.215 91.135) (width 0.25) (layer F.Cu) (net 10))
 (segment (start 144.04 93.31) (end 141.04 90.31) (width 0.25) (layer F.Cu) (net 10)))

